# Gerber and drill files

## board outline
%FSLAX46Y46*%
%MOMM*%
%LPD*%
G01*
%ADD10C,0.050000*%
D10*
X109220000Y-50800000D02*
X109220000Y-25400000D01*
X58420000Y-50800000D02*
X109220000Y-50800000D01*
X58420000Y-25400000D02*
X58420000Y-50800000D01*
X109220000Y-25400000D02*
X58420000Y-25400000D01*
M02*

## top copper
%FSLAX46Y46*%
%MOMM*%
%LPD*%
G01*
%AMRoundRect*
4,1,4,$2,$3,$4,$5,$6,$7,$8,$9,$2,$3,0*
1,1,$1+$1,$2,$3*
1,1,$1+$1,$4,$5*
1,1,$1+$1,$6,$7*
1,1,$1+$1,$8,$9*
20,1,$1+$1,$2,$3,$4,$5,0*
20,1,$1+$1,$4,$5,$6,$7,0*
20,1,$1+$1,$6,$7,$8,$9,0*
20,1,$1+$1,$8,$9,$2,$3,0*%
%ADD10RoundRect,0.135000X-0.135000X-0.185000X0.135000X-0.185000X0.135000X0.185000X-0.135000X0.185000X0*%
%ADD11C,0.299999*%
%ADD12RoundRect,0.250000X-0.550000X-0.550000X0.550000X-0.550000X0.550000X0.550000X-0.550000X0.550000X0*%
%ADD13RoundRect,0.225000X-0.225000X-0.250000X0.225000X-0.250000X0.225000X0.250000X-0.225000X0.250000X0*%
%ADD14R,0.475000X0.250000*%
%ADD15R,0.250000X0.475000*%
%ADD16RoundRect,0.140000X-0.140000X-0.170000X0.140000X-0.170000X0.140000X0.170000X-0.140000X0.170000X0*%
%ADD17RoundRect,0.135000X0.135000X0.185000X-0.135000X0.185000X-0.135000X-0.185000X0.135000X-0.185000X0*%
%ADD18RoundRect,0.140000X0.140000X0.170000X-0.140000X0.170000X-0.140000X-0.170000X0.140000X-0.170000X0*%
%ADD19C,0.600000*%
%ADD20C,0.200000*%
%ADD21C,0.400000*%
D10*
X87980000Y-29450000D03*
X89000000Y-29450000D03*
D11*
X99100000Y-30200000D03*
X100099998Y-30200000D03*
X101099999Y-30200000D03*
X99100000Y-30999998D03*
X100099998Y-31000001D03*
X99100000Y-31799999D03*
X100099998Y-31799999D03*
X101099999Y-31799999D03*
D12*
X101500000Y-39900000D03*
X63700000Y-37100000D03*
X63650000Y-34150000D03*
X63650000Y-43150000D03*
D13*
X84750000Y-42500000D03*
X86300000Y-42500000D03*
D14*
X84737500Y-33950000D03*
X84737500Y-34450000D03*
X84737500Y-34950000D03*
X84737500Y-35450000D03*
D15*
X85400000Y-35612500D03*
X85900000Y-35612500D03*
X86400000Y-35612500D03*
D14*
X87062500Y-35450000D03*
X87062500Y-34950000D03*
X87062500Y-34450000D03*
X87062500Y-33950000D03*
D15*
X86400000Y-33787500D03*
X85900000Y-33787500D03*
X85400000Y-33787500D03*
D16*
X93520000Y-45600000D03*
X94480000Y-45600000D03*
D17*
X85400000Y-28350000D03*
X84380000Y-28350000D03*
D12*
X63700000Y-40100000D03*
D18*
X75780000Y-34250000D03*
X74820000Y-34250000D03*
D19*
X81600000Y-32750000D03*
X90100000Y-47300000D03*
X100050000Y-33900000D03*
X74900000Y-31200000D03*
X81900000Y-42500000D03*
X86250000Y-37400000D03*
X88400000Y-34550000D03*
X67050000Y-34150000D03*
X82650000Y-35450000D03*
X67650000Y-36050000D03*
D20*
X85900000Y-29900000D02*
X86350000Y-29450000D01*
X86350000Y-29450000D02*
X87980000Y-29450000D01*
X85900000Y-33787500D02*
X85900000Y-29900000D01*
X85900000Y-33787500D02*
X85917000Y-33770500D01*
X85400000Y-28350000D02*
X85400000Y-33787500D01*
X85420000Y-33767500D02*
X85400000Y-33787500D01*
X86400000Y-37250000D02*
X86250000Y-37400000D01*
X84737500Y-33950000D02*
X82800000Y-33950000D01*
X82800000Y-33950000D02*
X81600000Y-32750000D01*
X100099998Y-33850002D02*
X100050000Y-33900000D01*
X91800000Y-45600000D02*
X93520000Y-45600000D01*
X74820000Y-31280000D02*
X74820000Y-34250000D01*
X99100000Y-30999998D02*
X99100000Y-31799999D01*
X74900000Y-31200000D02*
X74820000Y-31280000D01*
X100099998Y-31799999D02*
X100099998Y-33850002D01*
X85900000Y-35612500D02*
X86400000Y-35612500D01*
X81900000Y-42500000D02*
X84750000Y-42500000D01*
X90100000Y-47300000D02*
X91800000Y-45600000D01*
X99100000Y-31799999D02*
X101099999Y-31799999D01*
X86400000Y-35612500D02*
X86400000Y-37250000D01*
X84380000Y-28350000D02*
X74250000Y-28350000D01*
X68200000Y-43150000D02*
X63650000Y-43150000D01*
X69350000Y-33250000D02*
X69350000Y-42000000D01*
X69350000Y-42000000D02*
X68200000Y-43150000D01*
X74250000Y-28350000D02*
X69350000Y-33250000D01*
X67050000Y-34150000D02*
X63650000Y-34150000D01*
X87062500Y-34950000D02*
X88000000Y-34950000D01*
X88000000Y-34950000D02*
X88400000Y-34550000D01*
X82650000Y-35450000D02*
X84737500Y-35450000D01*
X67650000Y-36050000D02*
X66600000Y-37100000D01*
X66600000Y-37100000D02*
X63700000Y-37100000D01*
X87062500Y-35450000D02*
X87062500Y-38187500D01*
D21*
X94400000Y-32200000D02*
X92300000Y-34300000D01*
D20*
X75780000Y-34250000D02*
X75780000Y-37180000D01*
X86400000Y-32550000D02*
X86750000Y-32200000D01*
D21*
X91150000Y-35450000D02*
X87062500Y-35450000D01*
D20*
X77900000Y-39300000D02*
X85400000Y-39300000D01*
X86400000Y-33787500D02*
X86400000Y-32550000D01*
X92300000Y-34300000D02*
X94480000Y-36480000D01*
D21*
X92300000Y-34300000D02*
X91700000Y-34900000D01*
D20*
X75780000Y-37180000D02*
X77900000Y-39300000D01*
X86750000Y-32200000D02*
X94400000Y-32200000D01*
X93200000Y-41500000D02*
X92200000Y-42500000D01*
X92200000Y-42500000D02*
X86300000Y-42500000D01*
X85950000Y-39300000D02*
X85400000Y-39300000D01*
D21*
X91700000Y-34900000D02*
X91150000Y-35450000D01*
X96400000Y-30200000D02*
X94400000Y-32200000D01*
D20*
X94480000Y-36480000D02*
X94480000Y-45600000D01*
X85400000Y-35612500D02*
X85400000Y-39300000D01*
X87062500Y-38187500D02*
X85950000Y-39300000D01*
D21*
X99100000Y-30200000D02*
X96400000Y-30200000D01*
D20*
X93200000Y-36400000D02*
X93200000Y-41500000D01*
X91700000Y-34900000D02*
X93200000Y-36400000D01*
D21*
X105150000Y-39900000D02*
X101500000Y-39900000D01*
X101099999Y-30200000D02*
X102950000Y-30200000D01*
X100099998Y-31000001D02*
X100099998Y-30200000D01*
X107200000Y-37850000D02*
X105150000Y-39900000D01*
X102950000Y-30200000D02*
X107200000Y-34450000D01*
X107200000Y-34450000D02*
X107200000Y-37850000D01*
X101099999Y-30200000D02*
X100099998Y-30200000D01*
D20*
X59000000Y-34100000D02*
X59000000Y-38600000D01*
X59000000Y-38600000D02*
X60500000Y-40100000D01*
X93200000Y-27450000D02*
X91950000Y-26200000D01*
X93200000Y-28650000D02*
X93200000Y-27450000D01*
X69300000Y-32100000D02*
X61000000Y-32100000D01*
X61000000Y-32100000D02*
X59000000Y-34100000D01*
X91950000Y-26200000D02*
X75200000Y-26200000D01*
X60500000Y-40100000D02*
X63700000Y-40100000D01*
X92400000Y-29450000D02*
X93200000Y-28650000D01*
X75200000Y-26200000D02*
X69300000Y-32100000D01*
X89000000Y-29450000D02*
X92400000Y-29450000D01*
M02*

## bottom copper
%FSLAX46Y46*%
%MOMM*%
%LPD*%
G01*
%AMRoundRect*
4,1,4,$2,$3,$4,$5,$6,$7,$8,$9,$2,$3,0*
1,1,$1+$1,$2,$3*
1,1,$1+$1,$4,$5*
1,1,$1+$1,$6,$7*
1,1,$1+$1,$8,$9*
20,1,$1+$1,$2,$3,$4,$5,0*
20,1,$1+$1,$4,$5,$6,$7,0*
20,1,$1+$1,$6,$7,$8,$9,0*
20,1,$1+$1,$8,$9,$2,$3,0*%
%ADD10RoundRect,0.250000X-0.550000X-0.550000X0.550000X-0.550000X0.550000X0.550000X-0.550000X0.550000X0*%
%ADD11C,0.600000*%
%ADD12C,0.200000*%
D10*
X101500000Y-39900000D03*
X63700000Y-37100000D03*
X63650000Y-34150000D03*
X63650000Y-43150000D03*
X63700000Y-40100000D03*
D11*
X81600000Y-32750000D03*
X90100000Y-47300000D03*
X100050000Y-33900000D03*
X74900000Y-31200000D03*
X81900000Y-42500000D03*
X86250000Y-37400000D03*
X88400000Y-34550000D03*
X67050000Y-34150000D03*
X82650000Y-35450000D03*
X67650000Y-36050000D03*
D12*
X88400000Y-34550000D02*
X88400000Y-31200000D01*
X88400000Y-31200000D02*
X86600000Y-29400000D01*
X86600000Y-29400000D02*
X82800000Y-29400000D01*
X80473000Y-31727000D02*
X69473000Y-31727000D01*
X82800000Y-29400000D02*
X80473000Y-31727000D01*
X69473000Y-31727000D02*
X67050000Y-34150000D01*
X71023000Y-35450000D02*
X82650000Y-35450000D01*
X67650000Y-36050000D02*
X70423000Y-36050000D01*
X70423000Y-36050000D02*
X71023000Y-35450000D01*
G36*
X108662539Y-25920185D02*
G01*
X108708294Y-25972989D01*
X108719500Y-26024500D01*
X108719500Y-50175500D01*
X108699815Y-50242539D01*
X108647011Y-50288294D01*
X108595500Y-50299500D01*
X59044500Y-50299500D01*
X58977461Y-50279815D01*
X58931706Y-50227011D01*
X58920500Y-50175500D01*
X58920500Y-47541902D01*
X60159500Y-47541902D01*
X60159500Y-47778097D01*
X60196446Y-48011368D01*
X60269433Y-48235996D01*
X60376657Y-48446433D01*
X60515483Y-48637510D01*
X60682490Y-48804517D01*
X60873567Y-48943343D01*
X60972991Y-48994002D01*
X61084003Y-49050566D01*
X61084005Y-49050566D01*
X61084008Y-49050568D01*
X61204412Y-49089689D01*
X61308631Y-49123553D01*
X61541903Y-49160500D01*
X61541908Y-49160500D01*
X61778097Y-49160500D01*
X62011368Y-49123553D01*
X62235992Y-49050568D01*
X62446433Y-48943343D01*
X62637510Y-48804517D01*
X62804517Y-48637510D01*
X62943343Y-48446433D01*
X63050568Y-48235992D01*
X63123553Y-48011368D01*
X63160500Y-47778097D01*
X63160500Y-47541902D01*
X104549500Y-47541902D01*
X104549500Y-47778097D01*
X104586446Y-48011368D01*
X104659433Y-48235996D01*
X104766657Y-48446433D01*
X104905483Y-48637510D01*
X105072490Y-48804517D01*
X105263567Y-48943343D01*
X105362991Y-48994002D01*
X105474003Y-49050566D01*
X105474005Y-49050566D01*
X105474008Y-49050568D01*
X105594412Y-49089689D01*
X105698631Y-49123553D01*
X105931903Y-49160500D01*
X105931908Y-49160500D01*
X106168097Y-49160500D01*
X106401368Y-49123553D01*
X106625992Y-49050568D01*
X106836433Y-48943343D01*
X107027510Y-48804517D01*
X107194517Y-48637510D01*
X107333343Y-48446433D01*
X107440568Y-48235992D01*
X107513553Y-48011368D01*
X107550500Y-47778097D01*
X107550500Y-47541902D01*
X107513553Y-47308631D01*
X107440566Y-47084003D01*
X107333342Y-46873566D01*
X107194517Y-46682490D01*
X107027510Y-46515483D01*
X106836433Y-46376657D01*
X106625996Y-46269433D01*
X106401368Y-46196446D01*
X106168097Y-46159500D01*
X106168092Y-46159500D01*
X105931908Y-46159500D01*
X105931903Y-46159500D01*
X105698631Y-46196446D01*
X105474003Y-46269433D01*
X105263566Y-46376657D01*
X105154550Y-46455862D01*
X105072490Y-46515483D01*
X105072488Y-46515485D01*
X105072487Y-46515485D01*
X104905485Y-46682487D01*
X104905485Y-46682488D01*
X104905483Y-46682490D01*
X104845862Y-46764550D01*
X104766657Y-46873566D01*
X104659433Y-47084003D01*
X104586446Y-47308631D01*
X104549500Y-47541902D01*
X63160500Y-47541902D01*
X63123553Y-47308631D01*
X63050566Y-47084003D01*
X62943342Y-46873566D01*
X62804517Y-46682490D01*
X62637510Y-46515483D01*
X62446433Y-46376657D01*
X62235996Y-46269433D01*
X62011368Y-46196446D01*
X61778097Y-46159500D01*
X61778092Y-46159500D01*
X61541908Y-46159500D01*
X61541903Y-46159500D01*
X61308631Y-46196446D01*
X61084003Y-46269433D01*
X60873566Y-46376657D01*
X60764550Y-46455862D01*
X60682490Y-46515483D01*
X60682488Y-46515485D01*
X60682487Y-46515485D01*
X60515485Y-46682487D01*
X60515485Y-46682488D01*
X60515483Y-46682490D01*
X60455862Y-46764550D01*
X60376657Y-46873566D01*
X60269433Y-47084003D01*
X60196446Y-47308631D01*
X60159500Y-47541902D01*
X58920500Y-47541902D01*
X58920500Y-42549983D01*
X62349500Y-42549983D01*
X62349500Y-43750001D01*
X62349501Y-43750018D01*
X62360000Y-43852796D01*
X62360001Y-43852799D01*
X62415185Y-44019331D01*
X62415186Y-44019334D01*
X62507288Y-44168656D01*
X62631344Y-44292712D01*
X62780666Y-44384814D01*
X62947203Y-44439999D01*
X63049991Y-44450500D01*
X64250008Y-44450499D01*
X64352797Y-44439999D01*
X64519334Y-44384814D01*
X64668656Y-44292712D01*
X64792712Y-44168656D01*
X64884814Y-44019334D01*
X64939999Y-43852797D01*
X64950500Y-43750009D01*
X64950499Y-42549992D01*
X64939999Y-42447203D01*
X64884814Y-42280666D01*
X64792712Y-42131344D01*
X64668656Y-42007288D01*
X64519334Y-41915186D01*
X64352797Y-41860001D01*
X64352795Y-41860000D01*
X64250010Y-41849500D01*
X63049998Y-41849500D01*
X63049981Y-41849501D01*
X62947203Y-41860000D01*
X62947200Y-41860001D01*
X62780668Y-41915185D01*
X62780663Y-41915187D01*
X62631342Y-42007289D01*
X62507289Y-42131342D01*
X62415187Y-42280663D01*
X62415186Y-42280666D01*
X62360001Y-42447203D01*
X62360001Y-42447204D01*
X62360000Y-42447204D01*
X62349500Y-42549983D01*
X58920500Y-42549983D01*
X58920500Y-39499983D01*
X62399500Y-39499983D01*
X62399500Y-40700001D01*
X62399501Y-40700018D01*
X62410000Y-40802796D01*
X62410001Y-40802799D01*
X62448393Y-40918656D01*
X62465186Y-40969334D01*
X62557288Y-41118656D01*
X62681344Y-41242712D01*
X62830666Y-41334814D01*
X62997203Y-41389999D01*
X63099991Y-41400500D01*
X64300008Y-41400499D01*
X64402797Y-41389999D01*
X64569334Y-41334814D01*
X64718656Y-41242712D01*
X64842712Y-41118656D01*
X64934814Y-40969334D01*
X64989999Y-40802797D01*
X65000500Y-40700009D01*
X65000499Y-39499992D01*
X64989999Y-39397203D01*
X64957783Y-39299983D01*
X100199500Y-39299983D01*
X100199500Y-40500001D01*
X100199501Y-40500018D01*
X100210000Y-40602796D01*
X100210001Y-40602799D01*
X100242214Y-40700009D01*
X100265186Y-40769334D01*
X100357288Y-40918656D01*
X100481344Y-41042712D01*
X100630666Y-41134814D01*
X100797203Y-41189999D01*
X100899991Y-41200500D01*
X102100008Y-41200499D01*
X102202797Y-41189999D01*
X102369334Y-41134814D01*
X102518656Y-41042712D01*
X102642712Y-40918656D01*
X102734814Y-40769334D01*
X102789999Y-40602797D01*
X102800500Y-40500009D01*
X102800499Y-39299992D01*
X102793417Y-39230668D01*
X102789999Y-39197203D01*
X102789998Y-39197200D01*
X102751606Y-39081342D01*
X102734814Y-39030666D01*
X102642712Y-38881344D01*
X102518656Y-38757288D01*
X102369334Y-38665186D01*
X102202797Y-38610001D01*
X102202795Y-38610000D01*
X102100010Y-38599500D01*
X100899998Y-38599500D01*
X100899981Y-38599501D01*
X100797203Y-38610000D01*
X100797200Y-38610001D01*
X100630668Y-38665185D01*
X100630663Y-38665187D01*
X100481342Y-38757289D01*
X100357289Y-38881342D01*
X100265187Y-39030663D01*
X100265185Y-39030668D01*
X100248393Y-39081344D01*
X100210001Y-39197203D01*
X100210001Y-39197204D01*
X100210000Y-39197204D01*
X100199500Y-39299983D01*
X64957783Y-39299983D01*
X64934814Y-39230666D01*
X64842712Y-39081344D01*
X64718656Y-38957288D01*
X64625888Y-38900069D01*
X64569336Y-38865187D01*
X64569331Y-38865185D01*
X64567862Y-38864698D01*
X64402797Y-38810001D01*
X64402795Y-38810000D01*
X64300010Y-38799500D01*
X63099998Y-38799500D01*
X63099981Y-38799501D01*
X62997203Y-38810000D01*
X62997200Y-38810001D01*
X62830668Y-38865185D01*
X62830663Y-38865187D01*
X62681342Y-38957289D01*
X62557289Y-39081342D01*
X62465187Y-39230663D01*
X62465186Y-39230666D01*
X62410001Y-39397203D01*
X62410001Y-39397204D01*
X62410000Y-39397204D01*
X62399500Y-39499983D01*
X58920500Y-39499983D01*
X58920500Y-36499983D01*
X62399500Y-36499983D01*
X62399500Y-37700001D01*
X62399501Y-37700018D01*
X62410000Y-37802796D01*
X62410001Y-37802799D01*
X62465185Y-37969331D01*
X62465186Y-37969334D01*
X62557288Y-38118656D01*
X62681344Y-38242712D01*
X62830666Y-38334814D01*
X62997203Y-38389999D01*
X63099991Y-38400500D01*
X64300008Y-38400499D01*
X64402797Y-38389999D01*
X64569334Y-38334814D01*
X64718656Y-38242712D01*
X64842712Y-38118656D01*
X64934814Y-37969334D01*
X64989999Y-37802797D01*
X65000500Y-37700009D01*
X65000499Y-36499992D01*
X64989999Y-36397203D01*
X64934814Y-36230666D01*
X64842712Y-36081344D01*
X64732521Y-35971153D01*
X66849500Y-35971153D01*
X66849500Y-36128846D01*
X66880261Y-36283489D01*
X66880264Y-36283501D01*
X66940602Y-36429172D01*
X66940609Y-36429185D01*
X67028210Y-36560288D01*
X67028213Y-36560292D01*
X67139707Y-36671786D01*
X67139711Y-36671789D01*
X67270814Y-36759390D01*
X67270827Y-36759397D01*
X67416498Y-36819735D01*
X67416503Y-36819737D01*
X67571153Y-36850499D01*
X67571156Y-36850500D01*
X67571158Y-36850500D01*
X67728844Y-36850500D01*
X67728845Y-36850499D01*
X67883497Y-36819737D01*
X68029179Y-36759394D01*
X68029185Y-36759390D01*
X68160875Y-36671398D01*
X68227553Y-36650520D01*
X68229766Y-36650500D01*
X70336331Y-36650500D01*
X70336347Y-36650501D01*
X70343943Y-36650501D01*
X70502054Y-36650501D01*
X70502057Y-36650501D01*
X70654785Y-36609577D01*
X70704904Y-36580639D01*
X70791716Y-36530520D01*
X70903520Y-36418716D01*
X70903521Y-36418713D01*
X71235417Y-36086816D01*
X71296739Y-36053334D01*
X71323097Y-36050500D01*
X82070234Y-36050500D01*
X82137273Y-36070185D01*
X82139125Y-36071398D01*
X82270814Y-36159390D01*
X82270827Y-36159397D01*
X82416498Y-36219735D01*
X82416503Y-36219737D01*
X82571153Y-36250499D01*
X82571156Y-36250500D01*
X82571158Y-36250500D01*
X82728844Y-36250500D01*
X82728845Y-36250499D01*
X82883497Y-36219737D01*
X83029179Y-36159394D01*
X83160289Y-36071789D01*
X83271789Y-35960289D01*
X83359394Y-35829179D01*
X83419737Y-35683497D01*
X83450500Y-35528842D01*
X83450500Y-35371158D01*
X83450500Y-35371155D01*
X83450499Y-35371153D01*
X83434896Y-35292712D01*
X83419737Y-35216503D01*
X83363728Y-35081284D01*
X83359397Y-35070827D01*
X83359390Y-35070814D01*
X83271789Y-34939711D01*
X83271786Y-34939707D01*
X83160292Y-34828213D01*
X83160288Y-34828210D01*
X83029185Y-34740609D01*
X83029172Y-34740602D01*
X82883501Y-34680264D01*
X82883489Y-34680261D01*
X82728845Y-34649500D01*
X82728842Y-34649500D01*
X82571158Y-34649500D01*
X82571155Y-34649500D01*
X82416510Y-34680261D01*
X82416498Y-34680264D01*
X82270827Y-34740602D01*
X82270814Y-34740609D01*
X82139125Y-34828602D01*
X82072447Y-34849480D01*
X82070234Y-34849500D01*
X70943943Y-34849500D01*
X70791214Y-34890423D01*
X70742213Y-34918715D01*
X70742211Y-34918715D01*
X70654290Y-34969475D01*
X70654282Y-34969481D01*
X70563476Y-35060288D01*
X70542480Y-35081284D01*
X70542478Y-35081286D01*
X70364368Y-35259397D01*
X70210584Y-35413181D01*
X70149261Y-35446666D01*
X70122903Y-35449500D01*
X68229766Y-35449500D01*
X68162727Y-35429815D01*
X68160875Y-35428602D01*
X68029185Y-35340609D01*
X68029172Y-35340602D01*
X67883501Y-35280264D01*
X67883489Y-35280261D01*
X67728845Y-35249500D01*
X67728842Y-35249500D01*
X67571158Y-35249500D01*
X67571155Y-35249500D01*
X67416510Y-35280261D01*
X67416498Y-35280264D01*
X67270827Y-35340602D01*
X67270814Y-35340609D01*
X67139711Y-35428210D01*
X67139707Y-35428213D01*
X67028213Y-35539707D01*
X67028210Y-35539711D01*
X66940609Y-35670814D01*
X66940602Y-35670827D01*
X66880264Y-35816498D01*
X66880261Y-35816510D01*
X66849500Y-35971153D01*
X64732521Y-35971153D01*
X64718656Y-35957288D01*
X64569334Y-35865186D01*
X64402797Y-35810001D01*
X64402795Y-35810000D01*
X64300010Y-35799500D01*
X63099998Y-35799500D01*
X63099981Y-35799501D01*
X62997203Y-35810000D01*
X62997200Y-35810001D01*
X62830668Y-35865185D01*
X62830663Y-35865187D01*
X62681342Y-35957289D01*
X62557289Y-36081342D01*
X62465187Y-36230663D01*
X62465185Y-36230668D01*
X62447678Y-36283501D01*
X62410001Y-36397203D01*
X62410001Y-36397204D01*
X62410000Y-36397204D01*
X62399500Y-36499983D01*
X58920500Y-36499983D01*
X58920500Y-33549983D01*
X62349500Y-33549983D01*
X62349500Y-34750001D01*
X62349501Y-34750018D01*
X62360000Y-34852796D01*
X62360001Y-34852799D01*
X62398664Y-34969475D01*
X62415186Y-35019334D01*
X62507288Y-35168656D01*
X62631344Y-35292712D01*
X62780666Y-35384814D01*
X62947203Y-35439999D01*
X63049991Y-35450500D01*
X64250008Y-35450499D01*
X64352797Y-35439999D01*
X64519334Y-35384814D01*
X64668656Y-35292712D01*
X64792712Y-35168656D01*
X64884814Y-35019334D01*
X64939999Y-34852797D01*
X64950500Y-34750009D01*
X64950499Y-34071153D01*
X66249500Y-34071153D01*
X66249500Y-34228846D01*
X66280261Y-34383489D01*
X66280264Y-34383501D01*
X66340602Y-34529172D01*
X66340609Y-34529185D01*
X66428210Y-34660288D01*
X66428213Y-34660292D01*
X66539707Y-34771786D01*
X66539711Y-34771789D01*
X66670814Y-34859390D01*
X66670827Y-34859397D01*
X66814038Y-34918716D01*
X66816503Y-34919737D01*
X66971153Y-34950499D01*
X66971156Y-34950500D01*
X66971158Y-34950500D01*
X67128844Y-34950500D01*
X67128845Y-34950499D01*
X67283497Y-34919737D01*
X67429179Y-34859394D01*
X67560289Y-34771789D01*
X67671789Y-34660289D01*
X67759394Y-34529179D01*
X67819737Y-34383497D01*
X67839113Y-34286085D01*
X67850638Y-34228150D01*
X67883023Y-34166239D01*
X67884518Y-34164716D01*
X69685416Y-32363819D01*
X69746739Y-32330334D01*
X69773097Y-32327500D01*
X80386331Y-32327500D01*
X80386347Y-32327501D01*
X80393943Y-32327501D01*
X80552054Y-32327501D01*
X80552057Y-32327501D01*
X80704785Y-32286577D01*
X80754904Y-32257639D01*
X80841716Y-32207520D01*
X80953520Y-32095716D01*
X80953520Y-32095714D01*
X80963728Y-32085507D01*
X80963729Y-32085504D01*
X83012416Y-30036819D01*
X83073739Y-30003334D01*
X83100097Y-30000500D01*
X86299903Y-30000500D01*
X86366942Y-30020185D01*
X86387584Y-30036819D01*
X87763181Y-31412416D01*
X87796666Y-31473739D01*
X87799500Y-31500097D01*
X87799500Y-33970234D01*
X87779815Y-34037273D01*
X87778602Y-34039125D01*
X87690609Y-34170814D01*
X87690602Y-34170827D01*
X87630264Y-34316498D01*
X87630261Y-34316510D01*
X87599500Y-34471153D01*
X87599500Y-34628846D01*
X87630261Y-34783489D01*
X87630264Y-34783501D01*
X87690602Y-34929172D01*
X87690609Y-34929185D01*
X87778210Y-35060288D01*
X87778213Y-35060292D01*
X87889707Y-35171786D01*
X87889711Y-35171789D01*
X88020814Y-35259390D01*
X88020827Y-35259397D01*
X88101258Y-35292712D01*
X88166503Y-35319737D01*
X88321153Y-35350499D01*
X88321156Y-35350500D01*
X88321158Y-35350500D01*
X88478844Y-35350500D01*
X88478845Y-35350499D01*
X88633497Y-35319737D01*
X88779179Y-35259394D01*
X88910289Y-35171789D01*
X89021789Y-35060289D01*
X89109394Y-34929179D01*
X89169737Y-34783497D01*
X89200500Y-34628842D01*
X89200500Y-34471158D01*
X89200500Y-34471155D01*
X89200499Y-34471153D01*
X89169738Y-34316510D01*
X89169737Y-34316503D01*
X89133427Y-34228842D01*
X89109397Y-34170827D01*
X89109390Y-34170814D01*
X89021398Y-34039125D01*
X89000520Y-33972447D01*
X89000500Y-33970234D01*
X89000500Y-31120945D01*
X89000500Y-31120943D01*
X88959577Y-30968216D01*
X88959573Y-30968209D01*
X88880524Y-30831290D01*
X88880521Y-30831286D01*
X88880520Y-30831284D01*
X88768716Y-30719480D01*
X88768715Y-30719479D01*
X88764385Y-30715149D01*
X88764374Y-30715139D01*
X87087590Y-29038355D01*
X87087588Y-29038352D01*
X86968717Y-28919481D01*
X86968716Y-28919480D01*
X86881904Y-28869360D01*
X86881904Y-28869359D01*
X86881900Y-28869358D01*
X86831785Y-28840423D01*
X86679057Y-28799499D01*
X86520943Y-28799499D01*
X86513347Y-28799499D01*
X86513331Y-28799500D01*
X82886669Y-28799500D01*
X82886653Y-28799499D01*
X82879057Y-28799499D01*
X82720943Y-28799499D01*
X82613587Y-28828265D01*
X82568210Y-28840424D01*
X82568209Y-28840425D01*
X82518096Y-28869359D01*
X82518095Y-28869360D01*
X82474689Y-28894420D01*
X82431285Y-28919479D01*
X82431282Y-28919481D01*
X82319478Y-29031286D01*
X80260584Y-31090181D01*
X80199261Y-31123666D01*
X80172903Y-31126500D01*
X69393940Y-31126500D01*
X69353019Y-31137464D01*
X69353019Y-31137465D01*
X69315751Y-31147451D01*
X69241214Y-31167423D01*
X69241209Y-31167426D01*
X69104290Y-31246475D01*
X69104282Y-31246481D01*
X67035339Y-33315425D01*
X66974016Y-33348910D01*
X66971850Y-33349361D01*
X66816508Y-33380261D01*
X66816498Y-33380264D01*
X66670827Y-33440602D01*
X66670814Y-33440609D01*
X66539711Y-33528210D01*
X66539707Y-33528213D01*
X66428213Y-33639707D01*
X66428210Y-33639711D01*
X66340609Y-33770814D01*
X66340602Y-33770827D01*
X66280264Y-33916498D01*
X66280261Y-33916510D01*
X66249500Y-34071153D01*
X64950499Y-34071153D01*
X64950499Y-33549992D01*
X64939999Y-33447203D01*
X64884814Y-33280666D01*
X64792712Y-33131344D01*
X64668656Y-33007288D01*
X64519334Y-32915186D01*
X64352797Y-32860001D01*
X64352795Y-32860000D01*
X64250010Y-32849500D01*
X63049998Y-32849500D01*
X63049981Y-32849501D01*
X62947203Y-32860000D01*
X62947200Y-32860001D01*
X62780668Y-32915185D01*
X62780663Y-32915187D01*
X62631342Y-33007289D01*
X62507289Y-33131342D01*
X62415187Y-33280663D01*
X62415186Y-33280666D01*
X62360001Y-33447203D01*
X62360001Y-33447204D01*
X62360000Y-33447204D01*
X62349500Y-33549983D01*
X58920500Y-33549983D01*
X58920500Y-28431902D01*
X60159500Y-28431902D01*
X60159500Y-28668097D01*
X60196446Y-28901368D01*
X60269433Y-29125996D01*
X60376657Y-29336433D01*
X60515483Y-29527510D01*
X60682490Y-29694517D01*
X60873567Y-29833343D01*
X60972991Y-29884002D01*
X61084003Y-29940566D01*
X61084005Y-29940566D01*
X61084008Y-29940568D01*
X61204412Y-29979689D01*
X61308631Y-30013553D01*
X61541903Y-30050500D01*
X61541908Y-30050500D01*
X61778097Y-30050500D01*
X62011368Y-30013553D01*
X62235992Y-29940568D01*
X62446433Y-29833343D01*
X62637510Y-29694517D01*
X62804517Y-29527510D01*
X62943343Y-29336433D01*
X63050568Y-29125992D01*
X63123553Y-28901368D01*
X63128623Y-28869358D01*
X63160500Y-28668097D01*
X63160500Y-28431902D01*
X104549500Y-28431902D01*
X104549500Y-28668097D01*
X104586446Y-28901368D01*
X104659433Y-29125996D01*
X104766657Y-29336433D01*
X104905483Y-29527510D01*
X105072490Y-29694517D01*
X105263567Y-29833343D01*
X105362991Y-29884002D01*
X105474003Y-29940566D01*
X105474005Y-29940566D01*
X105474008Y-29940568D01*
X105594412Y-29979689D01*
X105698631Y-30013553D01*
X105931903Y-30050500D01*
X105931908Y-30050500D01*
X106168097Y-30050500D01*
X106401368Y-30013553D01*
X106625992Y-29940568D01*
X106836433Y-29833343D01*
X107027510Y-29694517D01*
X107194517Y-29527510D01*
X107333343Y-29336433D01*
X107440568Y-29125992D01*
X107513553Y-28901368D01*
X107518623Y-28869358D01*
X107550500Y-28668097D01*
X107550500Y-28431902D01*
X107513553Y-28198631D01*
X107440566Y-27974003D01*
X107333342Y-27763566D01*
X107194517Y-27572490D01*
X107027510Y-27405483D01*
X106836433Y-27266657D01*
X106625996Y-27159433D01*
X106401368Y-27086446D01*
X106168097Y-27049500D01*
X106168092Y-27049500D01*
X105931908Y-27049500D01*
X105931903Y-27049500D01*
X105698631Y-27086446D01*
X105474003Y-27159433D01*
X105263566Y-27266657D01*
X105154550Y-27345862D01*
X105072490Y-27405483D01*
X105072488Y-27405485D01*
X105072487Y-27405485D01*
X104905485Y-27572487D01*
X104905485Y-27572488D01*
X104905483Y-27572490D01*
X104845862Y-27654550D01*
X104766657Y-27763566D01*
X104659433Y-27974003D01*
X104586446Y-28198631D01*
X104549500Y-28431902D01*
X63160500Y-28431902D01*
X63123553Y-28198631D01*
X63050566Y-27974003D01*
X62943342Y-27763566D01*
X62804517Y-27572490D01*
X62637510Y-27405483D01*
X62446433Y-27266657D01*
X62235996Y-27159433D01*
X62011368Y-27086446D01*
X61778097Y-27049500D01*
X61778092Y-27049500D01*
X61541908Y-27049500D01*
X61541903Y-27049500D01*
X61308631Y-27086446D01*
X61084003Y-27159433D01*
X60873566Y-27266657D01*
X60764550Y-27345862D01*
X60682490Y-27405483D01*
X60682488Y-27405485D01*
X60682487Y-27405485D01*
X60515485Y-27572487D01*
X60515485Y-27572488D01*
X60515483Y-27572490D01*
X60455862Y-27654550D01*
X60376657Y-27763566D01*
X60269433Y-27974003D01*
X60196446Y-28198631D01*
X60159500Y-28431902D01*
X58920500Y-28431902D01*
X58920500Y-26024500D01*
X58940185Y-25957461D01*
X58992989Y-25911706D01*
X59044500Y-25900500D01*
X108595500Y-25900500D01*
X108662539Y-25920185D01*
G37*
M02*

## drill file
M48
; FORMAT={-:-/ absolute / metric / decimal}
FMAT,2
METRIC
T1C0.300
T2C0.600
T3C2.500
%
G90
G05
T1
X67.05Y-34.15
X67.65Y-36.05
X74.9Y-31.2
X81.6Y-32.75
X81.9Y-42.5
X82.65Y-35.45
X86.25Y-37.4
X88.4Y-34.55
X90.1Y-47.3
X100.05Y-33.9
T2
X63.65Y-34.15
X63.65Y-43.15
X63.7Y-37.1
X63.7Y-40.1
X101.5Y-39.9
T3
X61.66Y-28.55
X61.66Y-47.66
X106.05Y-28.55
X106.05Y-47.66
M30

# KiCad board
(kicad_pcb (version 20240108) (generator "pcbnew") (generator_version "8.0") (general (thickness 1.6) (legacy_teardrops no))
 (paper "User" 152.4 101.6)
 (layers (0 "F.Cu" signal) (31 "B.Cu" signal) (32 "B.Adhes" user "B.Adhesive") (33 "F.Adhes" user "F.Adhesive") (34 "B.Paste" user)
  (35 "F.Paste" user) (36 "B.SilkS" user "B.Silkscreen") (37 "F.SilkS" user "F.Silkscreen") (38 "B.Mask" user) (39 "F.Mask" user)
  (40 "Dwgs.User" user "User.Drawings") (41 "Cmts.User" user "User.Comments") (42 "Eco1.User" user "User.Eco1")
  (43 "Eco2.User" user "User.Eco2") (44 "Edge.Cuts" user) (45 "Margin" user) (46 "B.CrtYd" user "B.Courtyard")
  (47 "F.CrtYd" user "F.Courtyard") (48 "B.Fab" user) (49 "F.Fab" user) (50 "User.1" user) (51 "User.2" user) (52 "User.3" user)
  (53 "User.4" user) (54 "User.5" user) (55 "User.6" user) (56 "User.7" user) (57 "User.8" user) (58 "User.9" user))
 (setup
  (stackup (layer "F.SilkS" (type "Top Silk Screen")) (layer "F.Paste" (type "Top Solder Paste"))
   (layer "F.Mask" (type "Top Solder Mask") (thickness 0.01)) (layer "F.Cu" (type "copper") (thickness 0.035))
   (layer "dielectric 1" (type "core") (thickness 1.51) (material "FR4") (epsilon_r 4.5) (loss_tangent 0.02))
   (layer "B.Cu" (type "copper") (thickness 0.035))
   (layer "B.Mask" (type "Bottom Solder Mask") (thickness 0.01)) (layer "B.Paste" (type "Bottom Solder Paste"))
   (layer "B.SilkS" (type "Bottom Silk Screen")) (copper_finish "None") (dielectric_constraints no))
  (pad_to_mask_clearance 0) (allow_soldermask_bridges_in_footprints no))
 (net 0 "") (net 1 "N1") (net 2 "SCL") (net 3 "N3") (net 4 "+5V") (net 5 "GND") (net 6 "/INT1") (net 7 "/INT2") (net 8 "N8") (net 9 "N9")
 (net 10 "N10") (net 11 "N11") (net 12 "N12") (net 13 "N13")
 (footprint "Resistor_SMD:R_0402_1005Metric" (layer "F.Cu") (at 88.49 29.45)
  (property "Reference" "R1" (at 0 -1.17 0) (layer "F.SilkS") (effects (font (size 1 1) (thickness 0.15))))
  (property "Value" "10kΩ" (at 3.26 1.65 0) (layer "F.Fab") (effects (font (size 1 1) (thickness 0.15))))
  (pad "1" smd roundrect (at -0.51 0) (size 0.54 0.64) (layers "F.Cu" "F.Paste" "F.Mask") (roundrect_rratio 0.25) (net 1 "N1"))
  (pad "2" smd roundrect (at 0.51 0) (size 0.54 0.64) (layers "F.Cu" "F.Paste" "F.Mask") (roundrect_rratio 0.25) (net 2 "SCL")))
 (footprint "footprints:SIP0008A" (layer "F.Cu") (at 100.099998 31.000001)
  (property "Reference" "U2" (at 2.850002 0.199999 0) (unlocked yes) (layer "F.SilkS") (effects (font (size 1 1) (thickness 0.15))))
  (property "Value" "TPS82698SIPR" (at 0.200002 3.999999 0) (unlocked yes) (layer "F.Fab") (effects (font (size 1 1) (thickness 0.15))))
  (pad "A1" smd circle (at -0.999998 -0.800001) (size 0.299999 0.299999) (layers "F.Cu" "F.Paste" "F.Mask") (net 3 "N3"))
  (pad "A2" smd circle (at 0 -0.800001) (size 0.299999 0.299999) (layers "F.Cu" "F.Paste" "F.Mask") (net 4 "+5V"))
  (pad "A3" smd circle (at 1.000001 -0.800001) (size 0.299999 0.299999) (layers "F.Cu" "F.Paste" "F.Mask") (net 4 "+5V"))
  (pad "B1" smd circle (at -0.999998 -0.000003) (size 0.299999 0.299999) (layers "F.Cu" "F.Paste" "F.Mask") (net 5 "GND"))
  (pad "B2" smd circle (at 0 0) (size 0.299999 0.299999) (layers "F.Cu" "F.Paste" "F.Mask") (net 4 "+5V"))
  (pad "C1" smd circle (at -0.999998 0.799998) (size 0.299999 0.299999) (layers "F.Cu" "F.Paste" "F.Mask") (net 5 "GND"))
  (pad "C2" smd circle (at 0 0.799998) (size 0.299999 0.299999) (layers "F.Cu" "F.Paste" "F.Mask") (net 5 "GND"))
  (pad "C3" smd circle (at 1.000001 0.799998) (size 0.299999 0.299999) (layers "F.Cu" "F.Paste" "F.Mask") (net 5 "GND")))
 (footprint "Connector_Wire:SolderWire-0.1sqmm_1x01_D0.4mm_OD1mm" (layer "F.Cu") (at 101.5 39.9)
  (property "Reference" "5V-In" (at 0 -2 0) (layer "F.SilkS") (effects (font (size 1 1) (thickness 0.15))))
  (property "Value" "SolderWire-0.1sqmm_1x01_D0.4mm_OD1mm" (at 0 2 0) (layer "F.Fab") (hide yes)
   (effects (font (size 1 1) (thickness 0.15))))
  (pad "1" thru_hole roundrect (at 0 0) (size 1.6 1.6) (drill 0.6) (layers "*.Cu" "*.Mask") (remove_unused_layers no)
   (roundrect_rratio 0.15625) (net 4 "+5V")))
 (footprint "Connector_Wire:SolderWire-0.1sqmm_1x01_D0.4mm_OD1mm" (layer "F.Cu") (at 63.7 37.1)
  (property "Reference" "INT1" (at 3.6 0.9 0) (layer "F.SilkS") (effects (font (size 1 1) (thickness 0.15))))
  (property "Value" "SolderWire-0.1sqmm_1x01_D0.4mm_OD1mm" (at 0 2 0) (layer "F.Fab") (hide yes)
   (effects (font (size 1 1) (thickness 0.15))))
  (pad "1" thru_hole roundrect (at 0 0) (size 1.6 1.6) (drill 0.6) (layers "*.Cu" "*.Mask") (remove_unused_layers no)
   (roundrect_rratio 0.15625) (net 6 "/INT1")))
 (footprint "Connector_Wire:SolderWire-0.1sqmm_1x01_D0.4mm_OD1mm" (layer "F.Cu") (at 63.65 34.15)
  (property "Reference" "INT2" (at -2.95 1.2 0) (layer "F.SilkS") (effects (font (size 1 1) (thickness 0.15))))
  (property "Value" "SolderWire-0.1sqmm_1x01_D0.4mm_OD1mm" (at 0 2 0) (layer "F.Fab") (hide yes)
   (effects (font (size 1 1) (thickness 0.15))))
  (pad "1" thru_hole roundrect (at 0 0) (size 1.6 1.6) (drill 0.6) (layers "*.Cu" "*.Mask") (remove_unused_layers no)
   (roundrect_rratio 0.15625) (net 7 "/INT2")))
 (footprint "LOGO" (layer "F.Cu") (at 76.2 45.72)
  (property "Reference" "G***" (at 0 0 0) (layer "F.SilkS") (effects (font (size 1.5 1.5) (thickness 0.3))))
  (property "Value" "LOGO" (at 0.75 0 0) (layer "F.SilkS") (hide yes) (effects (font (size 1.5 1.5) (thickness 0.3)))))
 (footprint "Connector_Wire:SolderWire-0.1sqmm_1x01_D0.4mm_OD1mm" (layer "F.Cu") (at 63.65 43.15)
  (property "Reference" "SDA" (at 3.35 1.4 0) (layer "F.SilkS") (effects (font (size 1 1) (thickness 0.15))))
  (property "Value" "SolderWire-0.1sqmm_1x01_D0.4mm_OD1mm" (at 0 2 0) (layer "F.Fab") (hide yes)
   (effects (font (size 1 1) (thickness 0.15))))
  (pad "1" thru_hole roundrect (at 0 0) (size 1.6 1.6) (drill 0.6) (layers "*.Cu" "*.Mask") (remove_unused_layers no)
   (roundrect_rratio 0.15625) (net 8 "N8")))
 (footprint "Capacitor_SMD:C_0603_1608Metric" (layer "F.Cu") (at 85.525 42.5)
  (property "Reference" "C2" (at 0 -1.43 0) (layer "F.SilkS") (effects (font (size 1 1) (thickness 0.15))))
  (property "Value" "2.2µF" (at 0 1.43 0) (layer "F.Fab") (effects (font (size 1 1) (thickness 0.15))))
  (pad "1" smd roundrect (at -0.775 0) (size 0.9 0.95) (layers "F.Cu" "F.Paste" "F.Mask") (roundrect_rratio 0.25) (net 5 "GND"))
  (pad "2" smd roundrect (at 0.775 0) (size 0.9 0.95) (layers "F.Cu" "F.Paste" "F.Mask") (roundrect_rratio 0.25) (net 3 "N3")))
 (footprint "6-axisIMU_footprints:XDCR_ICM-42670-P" (layer "F.Cu") (at 85.9 34.7)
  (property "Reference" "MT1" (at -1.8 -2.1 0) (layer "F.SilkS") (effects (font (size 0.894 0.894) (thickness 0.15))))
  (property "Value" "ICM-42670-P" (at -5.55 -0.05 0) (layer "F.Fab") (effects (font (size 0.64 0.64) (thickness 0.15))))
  (pad "1" smd rect (at -1.1625 -0.75) (size 0.475 0.25) (layers "F.Cu") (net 5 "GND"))
  (pad "2" smd rect (at -1.1625 -0.25) (size 0.475 0.25) (layers "F.Cu") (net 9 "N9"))
  (pad "3" smd rect (at -1.1625 0.25) (size 0.475 0.25) (layers "F.Cu") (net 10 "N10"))
  (pad "4" smd rect (at -1.1625 0.75) (size 0.475 0.25) (layers "F.Cu") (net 6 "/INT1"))
  (pad "5" smd rect (at -0.5 0.9125) (size 0.25 0.475) (layers "F.Cu") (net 3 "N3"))
  (pad "6" smd rect (at 0 0.9125) (size 0.25 0.475) (layers "F.Cu") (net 5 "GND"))
  (pad "7" smd rect (at 0.5 0.9125) (size 0.25 0.475) (layers "F.Cu") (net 5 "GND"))
  (pad "8" smd rect (at 1.1625 0.75) (size 0.475 0.25) (layers "F.Cu") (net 3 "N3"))
  (pad "9" smd rect (at 1.1625 0.25) (size 0.475 0.25) (layers "F.Cu") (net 7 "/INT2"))
  (pad "10" smd rect (at 1.1625 -0.25) (size 0.475 0.25) (layers "F.Cu") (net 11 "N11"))
  (pad "11" smd rect (at 1.1625 -0.75) (size 0.475 0.25) (layers "F.Cu") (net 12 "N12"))
  (pad "12" smd rect (at 0.5 -0.9125) (size 0.25 0.475) (layers "F.Cu") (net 3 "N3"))
  (pad "13" smd rect (at 0 -0.9125) (size 0.25 0.475) (layers "F.Cu") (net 1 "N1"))
  (pad "14" smd rect (at -0.5 -0.9125) (size 0.25 0.475) (layers "F.Cu") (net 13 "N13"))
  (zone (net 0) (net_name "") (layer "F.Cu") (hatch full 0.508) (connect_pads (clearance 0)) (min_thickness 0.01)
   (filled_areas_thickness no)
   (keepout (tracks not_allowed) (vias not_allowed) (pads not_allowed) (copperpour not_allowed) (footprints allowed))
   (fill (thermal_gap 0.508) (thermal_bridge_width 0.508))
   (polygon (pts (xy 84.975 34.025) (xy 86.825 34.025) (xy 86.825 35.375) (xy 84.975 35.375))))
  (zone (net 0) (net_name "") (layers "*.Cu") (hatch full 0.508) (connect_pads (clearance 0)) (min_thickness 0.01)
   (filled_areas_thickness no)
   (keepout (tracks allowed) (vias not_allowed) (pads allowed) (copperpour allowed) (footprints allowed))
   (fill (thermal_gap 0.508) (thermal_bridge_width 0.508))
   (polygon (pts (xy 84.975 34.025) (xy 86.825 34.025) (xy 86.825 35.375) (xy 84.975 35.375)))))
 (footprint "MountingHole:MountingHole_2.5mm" (layer "F.Cu") (at 61.66 47.66)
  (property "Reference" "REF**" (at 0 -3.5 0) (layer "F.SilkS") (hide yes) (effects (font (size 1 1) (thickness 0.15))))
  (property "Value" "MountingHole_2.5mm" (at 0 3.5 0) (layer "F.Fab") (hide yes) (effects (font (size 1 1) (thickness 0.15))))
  (pad "" np_thru_hole circle (at 0 0) (size 2.5 2.5) (drill 2.5) (layers "*.Cu" "*.Mask")))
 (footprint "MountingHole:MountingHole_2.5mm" (layer "F.Cu") (at 106.05 47.66)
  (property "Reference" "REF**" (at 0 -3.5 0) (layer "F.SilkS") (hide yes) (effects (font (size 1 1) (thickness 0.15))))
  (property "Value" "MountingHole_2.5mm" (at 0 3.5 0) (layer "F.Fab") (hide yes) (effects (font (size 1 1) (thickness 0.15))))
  (pad "" np_thru_hole circle (at 0 0) (size 2.5 2.5) (drill 2.5) (layers "F&B.Cu" "*.Mask")))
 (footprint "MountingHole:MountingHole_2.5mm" (layer "F.Cu") (at 106.05 28.55)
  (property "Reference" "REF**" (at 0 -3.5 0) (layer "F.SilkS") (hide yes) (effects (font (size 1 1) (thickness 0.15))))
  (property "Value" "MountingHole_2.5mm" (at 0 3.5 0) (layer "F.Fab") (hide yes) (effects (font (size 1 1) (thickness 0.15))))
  (pad "" np_thru_hole circle (at 0 0) (size 2.5 2.5) (drill 2.5) (layers "F&B.Cu" "*.Mask")))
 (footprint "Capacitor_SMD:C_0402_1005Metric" (layer "F.Cu") (at 94 45.6)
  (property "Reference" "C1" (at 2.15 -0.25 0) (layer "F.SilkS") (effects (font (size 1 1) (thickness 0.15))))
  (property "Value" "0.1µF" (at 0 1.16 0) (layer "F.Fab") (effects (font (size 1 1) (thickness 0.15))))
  (pad "1" smd roundrect (at -0.48 0) (size 0.56 0.62) (layers "F.Cu" "F.Paste" "F.Mask") (roundrect_rratio 0.25) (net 5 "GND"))
  (pad "2" smd roundrect (at 0.48 0) (size 0.56 0.62) (layers "F.Cu" "F.Paste" "F.Mask") (roundrect_rratio 0.25) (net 3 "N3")))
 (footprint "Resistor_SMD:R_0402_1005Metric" (layer "F.Cu") (at 84.89 28.35 180)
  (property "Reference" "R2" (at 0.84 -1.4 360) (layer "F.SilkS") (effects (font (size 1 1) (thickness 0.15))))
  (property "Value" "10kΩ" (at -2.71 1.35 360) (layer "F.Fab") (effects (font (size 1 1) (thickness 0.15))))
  (pad "1" smd roundrect (at -0.51 0 180) (size 0.54 0.64) (layers "F.Cu" "F.Paste" "F.Mask") (roundrect_rratio 0.25) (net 13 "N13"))
  (pad "2" smd roundrect (at 0.51 0 180) (size 0.54 0.64) (layers "F.Cu" "F.Paste" "F.Mask") (roundrect_rratio 0.25) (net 8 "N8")))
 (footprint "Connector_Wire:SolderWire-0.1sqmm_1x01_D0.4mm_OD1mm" (layer "F.Cu") (at 63.7 40.1)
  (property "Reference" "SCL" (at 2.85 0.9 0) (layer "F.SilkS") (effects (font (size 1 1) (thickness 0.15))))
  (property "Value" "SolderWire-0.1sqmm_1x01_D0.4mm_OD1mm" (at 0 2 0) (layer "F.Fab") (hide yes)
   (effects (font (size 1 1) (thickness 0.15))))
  (pad "1" thru_hole roundrect (at 0 0) (size 1.6 1.6) (drill 0.6) (layers "*.Cu" "*.Mask") (remove_unused_layers no)
   (roundrect_rratio 0.15625) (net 2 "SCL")))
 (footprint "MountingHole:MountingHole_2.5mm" (layer "F.Cu") (at 61.66 28.55)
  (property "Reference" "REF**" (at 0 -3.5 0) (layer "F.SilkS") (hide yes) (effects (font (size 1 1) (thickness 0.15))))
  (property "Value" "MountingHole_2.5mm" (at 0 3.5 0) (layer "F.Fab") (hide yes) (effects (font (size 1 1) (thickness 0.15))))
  (pad "" np_thru_hole circle (at 0 0) (size 2.5 2.5) (drill 2.5) (layers "F&B.Cu" "*.Mask")))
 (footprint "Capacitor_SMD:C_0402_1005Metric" (layer "F.Cu") (at 75.3 34.25 180)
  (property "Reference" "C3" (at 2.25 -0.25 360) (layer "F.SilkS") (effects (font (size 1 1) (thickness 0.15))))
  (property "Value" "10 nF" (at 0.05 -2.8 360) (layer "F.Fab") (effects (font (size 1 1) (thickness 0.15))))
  (pad "1" smd roundrect (at -0.48 0 180) (size 0.56 0.62) (layers "F.Cu" "F.Paste" "F.Mask") (roundrect_rratio 0.25) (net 3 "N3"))
  (pad "2" smd roundrect (at 0.48 0 180) (size 0.56 0.62) (layers "F.Cu" "F.Paste" "F.Mask") (roundrect_rratio 0.25) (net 5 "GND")))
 (gr_line (start 109.22 50.8) (end 109.22 25.4) (stroke (width 0.05) (type default)) (layer "Edge.Cuts"))
 (gr_line (start 58.42 50.8) (end 109.22 50.8) (stroke (width 0.05) (type default)) (layer "Edge.Cuts"))
 (gr_line (start 58.42 25.4) (end 58.42 50.8) (stroke (width 0.05) (type default)) (layer "Edge.Cuts"))
 (gr_line (start 109.22 25.4) (end 58.42 25.4) (stroke (width 0.05) (type default)) (layer "Edge.Cuts"))
 (segment (start 85.9 29.9) (end 86.35 29.45) (width 0.2) (layer "F.Cu") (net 1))
 (segment (start 86.35 29.45) (end 87.98 29.45) (width 0.2) (layer "F.Cu") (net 1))
 (segment (start 85.9 33.7875) (end 85.9 29.9) (width 0.2) (layer "F.Cu") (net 1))
 (segment (start 85.9 33.7875) (end 85.917 33.7705) (width 0.2) (layer "F.Cu") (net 1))
 (segment (start 85.4 28.35) (end 85.4 33.7875) (width 0.2) (layer "F.Cu") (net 13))
 (segment (start 85.42 33.7675) (end 85.4 33.7875) (width 0.2) (layer "F.Cu") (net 13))
 (segment (start 86.4 37.25) (end 86.25 37.4) (width 0.2) (layer "F.Cu") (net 5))
 (segment (start 84.7375 33.95) (end 82.8 33.95) (width 0.2) (layer "F.Cu") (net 5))
 (segment (start 82.8 33.95) (end 81.6 32.75) (width 0.2) (layer "F.Cu") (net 5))
 (segment (start 100.099998 33.850002) (end 100.05 33.9) (width 0.2) (layer "F.Cu") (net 5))
 (segment (start 91.8 45.6) (end 93.52 45.6) (width 0.2) (layer "F.Cu") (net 5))
 (segment (start 74.82 31.28) (end 74.82 34.25) (width 0.2) (layer "F.Cu") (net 5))
 (segment (start 99.1 30.999998) (end 99.1 31.799999) (width 0.2) (layer "F.Cu") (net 5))
 (segment (start 74.9 31.2) (end 74.82 31.28) (width 0.2) (layer "F.Cu") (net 5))
 (segment (start 100.099998 31.799999) (end 100.099998 33.850002) (width 0.2) (layer "F.Cu") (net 5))
 (segment (start 85.9 35.6125) (end 86.4 35.6125) (width 0.2) (layer "F.Cu") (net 5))
 (segment (start 81.9 42.5) (end 84.75 42.5) (width 0.2) (layer "F.Cu") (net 5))
 (segment (start 90.1 47.3) (end 91.8 45.6) (width 0.2) (layer "F.Cu") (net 5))
 (segment (start 99.1 31.799999) (end 101.099999 31.799999) (width 0.2) (layer "F.Cu") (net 5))
 (segment (start 86.4 35.6125) (end 86.4 37.25) (width 0.2) (layer "F.Cu") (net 5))
 (via (at 81.6 32.75) (size 0.6) (drill 0.3) (layers "F.Cu" "B.Cu") (free yes) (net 5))
 (via (at 90.1 47.3) (size 0.6) (drill 0.3) (layers "F.Cu" "B.Cu") (free yes) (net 5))
 (via (at 100.05 33.9) (size 0.6) (drill 0.3) (layers "F.Cu" "B.Cu") (free yes) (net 5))
 (via (at 74.9 31.2) (size 0.6) (drill 0.3) (layers "F.Cu" "B.Cu") (free yes) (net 5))
 (via (at 81.9 42.5) (size 0.6) (drill 0.3) (layers "F.Cu" "B.Cu") (free yes) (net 5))
 (via (at 86.25 37.4) (size 0.6) (drill 0.3) (layers "F.Cu" "B.Cu") (free yes) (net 5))
 (segment (start 84.38 28.35) (end 74.25 28.35) (width 0.2) (layer "F.Cu") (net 8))
 (segment (start 68.2 43.15) (end 63.65 43.15) (width 0.2) (layer "F.Cu") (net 8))
 (segment (start 69.35 33.25) (end 69.35 42) (width 0.2) (layer "F.Cu") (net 8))
 (segment (start 69.35 42) (end 68.2 43.15) (width 0.2) (layer "F.Cu") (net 8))
 (segment (start 74.25 28.35) (end 69.35 33.25) (width 0.2) (layer "F.Cu") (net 8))
 (segment (start 67.05 34.15) (end 63.65 34.15) (width 0.2) (layer "F.Cu") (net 7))
 (segment (start 87.0625 34.95) (end 88 34.95) (width 0.2) (layer "F.Cu") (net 7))
 (segment (start 88 34.95) (end 88.4 34.55) (width 0.2) (layer "F.Cu") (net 7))
 (via (at 88.4 34.55) (size 0.6) (drill 0.3) (layers "F.Cu" "B.Cu") (free yes) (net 7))
 (via (at 67.05 34.15) (size 0.6) (drill 0.3) (layers "F.Cu" "B.Cu") (free yes) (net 7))
 (segment (start 88.4 34.55) (end 88.4 31.2) (width 0.2) (layer "B.Cu") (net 7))
 (segment (start 88.4 31.2) (end 86.6 29.4) (width 0.2) (layer "B.Cu") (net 7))
 (segment (start 86.6 29.4) (end 82.8 29.4) (width 0.2) (layer "B.Cu") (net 7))
 (segment (start 80.473 31.727) (end 69.473 31.727) (width 0.2) (layer "B.Cu") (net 7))
 (segment (start 82.8 29.4) (end 80.473 31.727) (width 0.2) (layer "B.Cu") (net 7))
 (segment (start 69.473 31.727) (end 67.05 34.15) (width 0.2) (layer "B.Cu") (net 7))
 (segment (start 82.65 35.45) (end 84.7375 35.45) (width 0.2) (layer "F.Cu") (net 6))
 (segment (start 67.65 36.05) (end 66.6 37.1) (width 0.2) (layer "F.Cu") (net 6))
 (segment (start 66.6 37.1) (end 63.7 37.1) (width 0.2) (layer "F.Cu") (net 6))
 (via (at 82.65 35.45) (size 0.6) (drill 0.3) (layers "F.Cu" "B.Cu") (free yes) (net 6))
 (via (at 67.65 36.05) (size 0.6) (drill 0.3) (layers "F.Cu" "B.Cu") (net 6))
 (segment (start 71.023 35.45) (end 82.65 35.45) (width 0.2) (layer "B.Cu") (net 6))
 (segment (start 67.65 36.05) (end 70.423 36.05) (width 0.2) (layer "B.Cu") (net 6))
 (segment (start 70.423 36.05) (end 71.023 35.45) (width 0.2) (layer "B.Cu") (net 6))
 (segment (start 87.0625 35.45) (end 87.0625 38.1875) (width 0.2) (layer "F.Cu") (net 3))
 (segment (start 94.4 32.2) (end 92.3 34.3) (width 0.4) (layer "F.Cu") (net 3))
 (segment (start 75.78 34.25) (end 75.78 37.18) (width 0.2) (layer "F.Cu") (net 3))
 (segment (start 86.4 32.55) (end 86.75 32.2) (width 0.2) (layer "F.Cu") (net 3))
 (segment (start 91.15 35.45) (end 87.0625 35.45) (width 0.4) (layer "F.Cu") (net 3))
 (segment (start 77.9 39.3) (end 85.4 39.3) (width 0.2) (layer "F.Cu") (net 3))
 (segment (start 86.4 33.7875) (end 86.4 32.55) (width 0.2) (layer "F.Cu") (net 3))
 (segment (start 92.3 34.3) (end 94.48 36.48) (width 0.2) (layer "F.Cu") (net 3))
 (segment (start 92.3 34.3) (end 91.7 34.9) (width 0.4) (layer "F.Cu") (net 3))
 (segment (start 75.78 37.18) (end 77.9 39.3) (width 0.2) (layer "F.Cu") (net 3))
 (segment (start 86.75 32.2) (end 94.4 32.2) (width 0.2) (layer "F.Cu") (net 3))
 (segment (start 93.2 41.5) (end 92.2 42.5) (width 0.2) (layer "F.Cu") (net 3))
 (segment (start 92.2 42.5) (end 86.3 42.5) (width 0.2) (layer "F.Cu") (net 3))
 (segment (start 85.95 39.3) (end 85.4 39.3) (width 0.2) (layer "F.Cu") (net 3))
 (segment (start 91.7 34.9) (end 91.15 35.45) (width 0.4) (layer "F.Cu") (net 3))
 (segment (start 96.4 30.2) (end 94.4 32.2) (width 0.4) (layer "F.Cu") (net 3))
 (segment (start 94.48 36.48) (end 94.48 45.6) (width 0.2) (layer "F.Cu") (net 3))
 (segment (start 85.4 35.6125) (end 85.4 39.3) (width 0.2) (layer "F.Cu") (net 3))
 (segment (start 87.0625 38.1875) (end 85.95 39.3) (width 0.2) (layer "F.Cu") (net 3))
 (segment (start 99.1 30.2) (end 96.4 30.2) (width 0.4) (layer "F.Cu") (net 3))
 (segment (start 93.2 36.4) (end 93.2 41.5) (width 0.2) (layer "F.Cu") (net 3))
 (segment (start 91.7 34.9) (end 93.2 36.4) (width 0.2) (layer "F.Cu") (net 3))
 (segment (start 105.15 39.9) (end 101.5 39.9) (width 0.4) (layer "F.Cu") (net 4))
 (segment (start 101.099999 30.2) (end 102.95 30.2) (width 0.4) (layer "F.Cu") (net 4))
 (segment (start 100.099998 31.000001) (end 100.099998 30.2) (width 0.4) (layer "F.Cu") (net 4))
 (segment (start 107.2 37.85) (end 105.15 39.9) (width 0.4) (layer "F.Cu") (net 4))
 (segment (start 102.95 30.2) (end 107.2 34.45) (width 0.4) (layer "F.Cu") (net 4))
 (segment (start 107.2 34.45) (end 107.2 37.85) (width 0.4) (layer "F.Cu") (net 4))
 (segment (start 101.099999 30.2) (end 100.099998 30.2) (width 0.4) (layer "F.Cu") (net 4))
 (segment (start 59 34.1) (end 59 38.6) (width 0.2) (layer "F.Cu") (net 2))
 (segment (start 59 38.6) (end 60.5 40.1) (width 0.2) (layer "F.Cu") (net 2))
 (segment (start 93.2 27.45) (end 91.95 26.2) (width 0.2) (layer "F.Cu") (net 2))
 (segment (start 93.2 28.65) (end 93.2 27.45) (width 0.2) (layer "F.Cu") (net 2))
 (segment (start 69.3 32.1) (end 61 32.1) (width 0.2) (layer "F.Cu") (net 2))
 (segment (start 61 32.1) (end 59 34.1) (width 0.2) (layer "F.Cu") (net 2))
 (segment (start 91.95 26.2) (end 75.2 26.2) (width 0.2) (layer "F.Cu") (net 2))
 (segment (start 60.5 40.1) (end 63.7 40.1) (width 0.2) (layer "F.Cu") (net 2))
 (segment (start 92.4 29.45) (end 93.2 28.65) (width 0.2) (layer "F.Cu") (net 2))
 (segment (start 75.2 26.2) (end 69.3 32.1) (width 0.2) (layer "F.Cu") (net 2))
 (segment (start 89 29.45) (end 92.4 29.45) (width 0.2) (layer "F.Cu") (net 2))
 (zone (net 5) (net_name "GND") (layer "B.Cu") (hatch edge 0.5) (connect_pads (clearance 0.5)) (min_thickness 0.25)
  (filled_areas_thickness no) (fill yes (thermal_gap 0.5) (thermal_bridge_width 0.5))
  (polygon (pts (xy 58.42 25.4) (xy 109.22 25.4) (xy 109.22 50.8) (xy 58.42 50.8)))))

